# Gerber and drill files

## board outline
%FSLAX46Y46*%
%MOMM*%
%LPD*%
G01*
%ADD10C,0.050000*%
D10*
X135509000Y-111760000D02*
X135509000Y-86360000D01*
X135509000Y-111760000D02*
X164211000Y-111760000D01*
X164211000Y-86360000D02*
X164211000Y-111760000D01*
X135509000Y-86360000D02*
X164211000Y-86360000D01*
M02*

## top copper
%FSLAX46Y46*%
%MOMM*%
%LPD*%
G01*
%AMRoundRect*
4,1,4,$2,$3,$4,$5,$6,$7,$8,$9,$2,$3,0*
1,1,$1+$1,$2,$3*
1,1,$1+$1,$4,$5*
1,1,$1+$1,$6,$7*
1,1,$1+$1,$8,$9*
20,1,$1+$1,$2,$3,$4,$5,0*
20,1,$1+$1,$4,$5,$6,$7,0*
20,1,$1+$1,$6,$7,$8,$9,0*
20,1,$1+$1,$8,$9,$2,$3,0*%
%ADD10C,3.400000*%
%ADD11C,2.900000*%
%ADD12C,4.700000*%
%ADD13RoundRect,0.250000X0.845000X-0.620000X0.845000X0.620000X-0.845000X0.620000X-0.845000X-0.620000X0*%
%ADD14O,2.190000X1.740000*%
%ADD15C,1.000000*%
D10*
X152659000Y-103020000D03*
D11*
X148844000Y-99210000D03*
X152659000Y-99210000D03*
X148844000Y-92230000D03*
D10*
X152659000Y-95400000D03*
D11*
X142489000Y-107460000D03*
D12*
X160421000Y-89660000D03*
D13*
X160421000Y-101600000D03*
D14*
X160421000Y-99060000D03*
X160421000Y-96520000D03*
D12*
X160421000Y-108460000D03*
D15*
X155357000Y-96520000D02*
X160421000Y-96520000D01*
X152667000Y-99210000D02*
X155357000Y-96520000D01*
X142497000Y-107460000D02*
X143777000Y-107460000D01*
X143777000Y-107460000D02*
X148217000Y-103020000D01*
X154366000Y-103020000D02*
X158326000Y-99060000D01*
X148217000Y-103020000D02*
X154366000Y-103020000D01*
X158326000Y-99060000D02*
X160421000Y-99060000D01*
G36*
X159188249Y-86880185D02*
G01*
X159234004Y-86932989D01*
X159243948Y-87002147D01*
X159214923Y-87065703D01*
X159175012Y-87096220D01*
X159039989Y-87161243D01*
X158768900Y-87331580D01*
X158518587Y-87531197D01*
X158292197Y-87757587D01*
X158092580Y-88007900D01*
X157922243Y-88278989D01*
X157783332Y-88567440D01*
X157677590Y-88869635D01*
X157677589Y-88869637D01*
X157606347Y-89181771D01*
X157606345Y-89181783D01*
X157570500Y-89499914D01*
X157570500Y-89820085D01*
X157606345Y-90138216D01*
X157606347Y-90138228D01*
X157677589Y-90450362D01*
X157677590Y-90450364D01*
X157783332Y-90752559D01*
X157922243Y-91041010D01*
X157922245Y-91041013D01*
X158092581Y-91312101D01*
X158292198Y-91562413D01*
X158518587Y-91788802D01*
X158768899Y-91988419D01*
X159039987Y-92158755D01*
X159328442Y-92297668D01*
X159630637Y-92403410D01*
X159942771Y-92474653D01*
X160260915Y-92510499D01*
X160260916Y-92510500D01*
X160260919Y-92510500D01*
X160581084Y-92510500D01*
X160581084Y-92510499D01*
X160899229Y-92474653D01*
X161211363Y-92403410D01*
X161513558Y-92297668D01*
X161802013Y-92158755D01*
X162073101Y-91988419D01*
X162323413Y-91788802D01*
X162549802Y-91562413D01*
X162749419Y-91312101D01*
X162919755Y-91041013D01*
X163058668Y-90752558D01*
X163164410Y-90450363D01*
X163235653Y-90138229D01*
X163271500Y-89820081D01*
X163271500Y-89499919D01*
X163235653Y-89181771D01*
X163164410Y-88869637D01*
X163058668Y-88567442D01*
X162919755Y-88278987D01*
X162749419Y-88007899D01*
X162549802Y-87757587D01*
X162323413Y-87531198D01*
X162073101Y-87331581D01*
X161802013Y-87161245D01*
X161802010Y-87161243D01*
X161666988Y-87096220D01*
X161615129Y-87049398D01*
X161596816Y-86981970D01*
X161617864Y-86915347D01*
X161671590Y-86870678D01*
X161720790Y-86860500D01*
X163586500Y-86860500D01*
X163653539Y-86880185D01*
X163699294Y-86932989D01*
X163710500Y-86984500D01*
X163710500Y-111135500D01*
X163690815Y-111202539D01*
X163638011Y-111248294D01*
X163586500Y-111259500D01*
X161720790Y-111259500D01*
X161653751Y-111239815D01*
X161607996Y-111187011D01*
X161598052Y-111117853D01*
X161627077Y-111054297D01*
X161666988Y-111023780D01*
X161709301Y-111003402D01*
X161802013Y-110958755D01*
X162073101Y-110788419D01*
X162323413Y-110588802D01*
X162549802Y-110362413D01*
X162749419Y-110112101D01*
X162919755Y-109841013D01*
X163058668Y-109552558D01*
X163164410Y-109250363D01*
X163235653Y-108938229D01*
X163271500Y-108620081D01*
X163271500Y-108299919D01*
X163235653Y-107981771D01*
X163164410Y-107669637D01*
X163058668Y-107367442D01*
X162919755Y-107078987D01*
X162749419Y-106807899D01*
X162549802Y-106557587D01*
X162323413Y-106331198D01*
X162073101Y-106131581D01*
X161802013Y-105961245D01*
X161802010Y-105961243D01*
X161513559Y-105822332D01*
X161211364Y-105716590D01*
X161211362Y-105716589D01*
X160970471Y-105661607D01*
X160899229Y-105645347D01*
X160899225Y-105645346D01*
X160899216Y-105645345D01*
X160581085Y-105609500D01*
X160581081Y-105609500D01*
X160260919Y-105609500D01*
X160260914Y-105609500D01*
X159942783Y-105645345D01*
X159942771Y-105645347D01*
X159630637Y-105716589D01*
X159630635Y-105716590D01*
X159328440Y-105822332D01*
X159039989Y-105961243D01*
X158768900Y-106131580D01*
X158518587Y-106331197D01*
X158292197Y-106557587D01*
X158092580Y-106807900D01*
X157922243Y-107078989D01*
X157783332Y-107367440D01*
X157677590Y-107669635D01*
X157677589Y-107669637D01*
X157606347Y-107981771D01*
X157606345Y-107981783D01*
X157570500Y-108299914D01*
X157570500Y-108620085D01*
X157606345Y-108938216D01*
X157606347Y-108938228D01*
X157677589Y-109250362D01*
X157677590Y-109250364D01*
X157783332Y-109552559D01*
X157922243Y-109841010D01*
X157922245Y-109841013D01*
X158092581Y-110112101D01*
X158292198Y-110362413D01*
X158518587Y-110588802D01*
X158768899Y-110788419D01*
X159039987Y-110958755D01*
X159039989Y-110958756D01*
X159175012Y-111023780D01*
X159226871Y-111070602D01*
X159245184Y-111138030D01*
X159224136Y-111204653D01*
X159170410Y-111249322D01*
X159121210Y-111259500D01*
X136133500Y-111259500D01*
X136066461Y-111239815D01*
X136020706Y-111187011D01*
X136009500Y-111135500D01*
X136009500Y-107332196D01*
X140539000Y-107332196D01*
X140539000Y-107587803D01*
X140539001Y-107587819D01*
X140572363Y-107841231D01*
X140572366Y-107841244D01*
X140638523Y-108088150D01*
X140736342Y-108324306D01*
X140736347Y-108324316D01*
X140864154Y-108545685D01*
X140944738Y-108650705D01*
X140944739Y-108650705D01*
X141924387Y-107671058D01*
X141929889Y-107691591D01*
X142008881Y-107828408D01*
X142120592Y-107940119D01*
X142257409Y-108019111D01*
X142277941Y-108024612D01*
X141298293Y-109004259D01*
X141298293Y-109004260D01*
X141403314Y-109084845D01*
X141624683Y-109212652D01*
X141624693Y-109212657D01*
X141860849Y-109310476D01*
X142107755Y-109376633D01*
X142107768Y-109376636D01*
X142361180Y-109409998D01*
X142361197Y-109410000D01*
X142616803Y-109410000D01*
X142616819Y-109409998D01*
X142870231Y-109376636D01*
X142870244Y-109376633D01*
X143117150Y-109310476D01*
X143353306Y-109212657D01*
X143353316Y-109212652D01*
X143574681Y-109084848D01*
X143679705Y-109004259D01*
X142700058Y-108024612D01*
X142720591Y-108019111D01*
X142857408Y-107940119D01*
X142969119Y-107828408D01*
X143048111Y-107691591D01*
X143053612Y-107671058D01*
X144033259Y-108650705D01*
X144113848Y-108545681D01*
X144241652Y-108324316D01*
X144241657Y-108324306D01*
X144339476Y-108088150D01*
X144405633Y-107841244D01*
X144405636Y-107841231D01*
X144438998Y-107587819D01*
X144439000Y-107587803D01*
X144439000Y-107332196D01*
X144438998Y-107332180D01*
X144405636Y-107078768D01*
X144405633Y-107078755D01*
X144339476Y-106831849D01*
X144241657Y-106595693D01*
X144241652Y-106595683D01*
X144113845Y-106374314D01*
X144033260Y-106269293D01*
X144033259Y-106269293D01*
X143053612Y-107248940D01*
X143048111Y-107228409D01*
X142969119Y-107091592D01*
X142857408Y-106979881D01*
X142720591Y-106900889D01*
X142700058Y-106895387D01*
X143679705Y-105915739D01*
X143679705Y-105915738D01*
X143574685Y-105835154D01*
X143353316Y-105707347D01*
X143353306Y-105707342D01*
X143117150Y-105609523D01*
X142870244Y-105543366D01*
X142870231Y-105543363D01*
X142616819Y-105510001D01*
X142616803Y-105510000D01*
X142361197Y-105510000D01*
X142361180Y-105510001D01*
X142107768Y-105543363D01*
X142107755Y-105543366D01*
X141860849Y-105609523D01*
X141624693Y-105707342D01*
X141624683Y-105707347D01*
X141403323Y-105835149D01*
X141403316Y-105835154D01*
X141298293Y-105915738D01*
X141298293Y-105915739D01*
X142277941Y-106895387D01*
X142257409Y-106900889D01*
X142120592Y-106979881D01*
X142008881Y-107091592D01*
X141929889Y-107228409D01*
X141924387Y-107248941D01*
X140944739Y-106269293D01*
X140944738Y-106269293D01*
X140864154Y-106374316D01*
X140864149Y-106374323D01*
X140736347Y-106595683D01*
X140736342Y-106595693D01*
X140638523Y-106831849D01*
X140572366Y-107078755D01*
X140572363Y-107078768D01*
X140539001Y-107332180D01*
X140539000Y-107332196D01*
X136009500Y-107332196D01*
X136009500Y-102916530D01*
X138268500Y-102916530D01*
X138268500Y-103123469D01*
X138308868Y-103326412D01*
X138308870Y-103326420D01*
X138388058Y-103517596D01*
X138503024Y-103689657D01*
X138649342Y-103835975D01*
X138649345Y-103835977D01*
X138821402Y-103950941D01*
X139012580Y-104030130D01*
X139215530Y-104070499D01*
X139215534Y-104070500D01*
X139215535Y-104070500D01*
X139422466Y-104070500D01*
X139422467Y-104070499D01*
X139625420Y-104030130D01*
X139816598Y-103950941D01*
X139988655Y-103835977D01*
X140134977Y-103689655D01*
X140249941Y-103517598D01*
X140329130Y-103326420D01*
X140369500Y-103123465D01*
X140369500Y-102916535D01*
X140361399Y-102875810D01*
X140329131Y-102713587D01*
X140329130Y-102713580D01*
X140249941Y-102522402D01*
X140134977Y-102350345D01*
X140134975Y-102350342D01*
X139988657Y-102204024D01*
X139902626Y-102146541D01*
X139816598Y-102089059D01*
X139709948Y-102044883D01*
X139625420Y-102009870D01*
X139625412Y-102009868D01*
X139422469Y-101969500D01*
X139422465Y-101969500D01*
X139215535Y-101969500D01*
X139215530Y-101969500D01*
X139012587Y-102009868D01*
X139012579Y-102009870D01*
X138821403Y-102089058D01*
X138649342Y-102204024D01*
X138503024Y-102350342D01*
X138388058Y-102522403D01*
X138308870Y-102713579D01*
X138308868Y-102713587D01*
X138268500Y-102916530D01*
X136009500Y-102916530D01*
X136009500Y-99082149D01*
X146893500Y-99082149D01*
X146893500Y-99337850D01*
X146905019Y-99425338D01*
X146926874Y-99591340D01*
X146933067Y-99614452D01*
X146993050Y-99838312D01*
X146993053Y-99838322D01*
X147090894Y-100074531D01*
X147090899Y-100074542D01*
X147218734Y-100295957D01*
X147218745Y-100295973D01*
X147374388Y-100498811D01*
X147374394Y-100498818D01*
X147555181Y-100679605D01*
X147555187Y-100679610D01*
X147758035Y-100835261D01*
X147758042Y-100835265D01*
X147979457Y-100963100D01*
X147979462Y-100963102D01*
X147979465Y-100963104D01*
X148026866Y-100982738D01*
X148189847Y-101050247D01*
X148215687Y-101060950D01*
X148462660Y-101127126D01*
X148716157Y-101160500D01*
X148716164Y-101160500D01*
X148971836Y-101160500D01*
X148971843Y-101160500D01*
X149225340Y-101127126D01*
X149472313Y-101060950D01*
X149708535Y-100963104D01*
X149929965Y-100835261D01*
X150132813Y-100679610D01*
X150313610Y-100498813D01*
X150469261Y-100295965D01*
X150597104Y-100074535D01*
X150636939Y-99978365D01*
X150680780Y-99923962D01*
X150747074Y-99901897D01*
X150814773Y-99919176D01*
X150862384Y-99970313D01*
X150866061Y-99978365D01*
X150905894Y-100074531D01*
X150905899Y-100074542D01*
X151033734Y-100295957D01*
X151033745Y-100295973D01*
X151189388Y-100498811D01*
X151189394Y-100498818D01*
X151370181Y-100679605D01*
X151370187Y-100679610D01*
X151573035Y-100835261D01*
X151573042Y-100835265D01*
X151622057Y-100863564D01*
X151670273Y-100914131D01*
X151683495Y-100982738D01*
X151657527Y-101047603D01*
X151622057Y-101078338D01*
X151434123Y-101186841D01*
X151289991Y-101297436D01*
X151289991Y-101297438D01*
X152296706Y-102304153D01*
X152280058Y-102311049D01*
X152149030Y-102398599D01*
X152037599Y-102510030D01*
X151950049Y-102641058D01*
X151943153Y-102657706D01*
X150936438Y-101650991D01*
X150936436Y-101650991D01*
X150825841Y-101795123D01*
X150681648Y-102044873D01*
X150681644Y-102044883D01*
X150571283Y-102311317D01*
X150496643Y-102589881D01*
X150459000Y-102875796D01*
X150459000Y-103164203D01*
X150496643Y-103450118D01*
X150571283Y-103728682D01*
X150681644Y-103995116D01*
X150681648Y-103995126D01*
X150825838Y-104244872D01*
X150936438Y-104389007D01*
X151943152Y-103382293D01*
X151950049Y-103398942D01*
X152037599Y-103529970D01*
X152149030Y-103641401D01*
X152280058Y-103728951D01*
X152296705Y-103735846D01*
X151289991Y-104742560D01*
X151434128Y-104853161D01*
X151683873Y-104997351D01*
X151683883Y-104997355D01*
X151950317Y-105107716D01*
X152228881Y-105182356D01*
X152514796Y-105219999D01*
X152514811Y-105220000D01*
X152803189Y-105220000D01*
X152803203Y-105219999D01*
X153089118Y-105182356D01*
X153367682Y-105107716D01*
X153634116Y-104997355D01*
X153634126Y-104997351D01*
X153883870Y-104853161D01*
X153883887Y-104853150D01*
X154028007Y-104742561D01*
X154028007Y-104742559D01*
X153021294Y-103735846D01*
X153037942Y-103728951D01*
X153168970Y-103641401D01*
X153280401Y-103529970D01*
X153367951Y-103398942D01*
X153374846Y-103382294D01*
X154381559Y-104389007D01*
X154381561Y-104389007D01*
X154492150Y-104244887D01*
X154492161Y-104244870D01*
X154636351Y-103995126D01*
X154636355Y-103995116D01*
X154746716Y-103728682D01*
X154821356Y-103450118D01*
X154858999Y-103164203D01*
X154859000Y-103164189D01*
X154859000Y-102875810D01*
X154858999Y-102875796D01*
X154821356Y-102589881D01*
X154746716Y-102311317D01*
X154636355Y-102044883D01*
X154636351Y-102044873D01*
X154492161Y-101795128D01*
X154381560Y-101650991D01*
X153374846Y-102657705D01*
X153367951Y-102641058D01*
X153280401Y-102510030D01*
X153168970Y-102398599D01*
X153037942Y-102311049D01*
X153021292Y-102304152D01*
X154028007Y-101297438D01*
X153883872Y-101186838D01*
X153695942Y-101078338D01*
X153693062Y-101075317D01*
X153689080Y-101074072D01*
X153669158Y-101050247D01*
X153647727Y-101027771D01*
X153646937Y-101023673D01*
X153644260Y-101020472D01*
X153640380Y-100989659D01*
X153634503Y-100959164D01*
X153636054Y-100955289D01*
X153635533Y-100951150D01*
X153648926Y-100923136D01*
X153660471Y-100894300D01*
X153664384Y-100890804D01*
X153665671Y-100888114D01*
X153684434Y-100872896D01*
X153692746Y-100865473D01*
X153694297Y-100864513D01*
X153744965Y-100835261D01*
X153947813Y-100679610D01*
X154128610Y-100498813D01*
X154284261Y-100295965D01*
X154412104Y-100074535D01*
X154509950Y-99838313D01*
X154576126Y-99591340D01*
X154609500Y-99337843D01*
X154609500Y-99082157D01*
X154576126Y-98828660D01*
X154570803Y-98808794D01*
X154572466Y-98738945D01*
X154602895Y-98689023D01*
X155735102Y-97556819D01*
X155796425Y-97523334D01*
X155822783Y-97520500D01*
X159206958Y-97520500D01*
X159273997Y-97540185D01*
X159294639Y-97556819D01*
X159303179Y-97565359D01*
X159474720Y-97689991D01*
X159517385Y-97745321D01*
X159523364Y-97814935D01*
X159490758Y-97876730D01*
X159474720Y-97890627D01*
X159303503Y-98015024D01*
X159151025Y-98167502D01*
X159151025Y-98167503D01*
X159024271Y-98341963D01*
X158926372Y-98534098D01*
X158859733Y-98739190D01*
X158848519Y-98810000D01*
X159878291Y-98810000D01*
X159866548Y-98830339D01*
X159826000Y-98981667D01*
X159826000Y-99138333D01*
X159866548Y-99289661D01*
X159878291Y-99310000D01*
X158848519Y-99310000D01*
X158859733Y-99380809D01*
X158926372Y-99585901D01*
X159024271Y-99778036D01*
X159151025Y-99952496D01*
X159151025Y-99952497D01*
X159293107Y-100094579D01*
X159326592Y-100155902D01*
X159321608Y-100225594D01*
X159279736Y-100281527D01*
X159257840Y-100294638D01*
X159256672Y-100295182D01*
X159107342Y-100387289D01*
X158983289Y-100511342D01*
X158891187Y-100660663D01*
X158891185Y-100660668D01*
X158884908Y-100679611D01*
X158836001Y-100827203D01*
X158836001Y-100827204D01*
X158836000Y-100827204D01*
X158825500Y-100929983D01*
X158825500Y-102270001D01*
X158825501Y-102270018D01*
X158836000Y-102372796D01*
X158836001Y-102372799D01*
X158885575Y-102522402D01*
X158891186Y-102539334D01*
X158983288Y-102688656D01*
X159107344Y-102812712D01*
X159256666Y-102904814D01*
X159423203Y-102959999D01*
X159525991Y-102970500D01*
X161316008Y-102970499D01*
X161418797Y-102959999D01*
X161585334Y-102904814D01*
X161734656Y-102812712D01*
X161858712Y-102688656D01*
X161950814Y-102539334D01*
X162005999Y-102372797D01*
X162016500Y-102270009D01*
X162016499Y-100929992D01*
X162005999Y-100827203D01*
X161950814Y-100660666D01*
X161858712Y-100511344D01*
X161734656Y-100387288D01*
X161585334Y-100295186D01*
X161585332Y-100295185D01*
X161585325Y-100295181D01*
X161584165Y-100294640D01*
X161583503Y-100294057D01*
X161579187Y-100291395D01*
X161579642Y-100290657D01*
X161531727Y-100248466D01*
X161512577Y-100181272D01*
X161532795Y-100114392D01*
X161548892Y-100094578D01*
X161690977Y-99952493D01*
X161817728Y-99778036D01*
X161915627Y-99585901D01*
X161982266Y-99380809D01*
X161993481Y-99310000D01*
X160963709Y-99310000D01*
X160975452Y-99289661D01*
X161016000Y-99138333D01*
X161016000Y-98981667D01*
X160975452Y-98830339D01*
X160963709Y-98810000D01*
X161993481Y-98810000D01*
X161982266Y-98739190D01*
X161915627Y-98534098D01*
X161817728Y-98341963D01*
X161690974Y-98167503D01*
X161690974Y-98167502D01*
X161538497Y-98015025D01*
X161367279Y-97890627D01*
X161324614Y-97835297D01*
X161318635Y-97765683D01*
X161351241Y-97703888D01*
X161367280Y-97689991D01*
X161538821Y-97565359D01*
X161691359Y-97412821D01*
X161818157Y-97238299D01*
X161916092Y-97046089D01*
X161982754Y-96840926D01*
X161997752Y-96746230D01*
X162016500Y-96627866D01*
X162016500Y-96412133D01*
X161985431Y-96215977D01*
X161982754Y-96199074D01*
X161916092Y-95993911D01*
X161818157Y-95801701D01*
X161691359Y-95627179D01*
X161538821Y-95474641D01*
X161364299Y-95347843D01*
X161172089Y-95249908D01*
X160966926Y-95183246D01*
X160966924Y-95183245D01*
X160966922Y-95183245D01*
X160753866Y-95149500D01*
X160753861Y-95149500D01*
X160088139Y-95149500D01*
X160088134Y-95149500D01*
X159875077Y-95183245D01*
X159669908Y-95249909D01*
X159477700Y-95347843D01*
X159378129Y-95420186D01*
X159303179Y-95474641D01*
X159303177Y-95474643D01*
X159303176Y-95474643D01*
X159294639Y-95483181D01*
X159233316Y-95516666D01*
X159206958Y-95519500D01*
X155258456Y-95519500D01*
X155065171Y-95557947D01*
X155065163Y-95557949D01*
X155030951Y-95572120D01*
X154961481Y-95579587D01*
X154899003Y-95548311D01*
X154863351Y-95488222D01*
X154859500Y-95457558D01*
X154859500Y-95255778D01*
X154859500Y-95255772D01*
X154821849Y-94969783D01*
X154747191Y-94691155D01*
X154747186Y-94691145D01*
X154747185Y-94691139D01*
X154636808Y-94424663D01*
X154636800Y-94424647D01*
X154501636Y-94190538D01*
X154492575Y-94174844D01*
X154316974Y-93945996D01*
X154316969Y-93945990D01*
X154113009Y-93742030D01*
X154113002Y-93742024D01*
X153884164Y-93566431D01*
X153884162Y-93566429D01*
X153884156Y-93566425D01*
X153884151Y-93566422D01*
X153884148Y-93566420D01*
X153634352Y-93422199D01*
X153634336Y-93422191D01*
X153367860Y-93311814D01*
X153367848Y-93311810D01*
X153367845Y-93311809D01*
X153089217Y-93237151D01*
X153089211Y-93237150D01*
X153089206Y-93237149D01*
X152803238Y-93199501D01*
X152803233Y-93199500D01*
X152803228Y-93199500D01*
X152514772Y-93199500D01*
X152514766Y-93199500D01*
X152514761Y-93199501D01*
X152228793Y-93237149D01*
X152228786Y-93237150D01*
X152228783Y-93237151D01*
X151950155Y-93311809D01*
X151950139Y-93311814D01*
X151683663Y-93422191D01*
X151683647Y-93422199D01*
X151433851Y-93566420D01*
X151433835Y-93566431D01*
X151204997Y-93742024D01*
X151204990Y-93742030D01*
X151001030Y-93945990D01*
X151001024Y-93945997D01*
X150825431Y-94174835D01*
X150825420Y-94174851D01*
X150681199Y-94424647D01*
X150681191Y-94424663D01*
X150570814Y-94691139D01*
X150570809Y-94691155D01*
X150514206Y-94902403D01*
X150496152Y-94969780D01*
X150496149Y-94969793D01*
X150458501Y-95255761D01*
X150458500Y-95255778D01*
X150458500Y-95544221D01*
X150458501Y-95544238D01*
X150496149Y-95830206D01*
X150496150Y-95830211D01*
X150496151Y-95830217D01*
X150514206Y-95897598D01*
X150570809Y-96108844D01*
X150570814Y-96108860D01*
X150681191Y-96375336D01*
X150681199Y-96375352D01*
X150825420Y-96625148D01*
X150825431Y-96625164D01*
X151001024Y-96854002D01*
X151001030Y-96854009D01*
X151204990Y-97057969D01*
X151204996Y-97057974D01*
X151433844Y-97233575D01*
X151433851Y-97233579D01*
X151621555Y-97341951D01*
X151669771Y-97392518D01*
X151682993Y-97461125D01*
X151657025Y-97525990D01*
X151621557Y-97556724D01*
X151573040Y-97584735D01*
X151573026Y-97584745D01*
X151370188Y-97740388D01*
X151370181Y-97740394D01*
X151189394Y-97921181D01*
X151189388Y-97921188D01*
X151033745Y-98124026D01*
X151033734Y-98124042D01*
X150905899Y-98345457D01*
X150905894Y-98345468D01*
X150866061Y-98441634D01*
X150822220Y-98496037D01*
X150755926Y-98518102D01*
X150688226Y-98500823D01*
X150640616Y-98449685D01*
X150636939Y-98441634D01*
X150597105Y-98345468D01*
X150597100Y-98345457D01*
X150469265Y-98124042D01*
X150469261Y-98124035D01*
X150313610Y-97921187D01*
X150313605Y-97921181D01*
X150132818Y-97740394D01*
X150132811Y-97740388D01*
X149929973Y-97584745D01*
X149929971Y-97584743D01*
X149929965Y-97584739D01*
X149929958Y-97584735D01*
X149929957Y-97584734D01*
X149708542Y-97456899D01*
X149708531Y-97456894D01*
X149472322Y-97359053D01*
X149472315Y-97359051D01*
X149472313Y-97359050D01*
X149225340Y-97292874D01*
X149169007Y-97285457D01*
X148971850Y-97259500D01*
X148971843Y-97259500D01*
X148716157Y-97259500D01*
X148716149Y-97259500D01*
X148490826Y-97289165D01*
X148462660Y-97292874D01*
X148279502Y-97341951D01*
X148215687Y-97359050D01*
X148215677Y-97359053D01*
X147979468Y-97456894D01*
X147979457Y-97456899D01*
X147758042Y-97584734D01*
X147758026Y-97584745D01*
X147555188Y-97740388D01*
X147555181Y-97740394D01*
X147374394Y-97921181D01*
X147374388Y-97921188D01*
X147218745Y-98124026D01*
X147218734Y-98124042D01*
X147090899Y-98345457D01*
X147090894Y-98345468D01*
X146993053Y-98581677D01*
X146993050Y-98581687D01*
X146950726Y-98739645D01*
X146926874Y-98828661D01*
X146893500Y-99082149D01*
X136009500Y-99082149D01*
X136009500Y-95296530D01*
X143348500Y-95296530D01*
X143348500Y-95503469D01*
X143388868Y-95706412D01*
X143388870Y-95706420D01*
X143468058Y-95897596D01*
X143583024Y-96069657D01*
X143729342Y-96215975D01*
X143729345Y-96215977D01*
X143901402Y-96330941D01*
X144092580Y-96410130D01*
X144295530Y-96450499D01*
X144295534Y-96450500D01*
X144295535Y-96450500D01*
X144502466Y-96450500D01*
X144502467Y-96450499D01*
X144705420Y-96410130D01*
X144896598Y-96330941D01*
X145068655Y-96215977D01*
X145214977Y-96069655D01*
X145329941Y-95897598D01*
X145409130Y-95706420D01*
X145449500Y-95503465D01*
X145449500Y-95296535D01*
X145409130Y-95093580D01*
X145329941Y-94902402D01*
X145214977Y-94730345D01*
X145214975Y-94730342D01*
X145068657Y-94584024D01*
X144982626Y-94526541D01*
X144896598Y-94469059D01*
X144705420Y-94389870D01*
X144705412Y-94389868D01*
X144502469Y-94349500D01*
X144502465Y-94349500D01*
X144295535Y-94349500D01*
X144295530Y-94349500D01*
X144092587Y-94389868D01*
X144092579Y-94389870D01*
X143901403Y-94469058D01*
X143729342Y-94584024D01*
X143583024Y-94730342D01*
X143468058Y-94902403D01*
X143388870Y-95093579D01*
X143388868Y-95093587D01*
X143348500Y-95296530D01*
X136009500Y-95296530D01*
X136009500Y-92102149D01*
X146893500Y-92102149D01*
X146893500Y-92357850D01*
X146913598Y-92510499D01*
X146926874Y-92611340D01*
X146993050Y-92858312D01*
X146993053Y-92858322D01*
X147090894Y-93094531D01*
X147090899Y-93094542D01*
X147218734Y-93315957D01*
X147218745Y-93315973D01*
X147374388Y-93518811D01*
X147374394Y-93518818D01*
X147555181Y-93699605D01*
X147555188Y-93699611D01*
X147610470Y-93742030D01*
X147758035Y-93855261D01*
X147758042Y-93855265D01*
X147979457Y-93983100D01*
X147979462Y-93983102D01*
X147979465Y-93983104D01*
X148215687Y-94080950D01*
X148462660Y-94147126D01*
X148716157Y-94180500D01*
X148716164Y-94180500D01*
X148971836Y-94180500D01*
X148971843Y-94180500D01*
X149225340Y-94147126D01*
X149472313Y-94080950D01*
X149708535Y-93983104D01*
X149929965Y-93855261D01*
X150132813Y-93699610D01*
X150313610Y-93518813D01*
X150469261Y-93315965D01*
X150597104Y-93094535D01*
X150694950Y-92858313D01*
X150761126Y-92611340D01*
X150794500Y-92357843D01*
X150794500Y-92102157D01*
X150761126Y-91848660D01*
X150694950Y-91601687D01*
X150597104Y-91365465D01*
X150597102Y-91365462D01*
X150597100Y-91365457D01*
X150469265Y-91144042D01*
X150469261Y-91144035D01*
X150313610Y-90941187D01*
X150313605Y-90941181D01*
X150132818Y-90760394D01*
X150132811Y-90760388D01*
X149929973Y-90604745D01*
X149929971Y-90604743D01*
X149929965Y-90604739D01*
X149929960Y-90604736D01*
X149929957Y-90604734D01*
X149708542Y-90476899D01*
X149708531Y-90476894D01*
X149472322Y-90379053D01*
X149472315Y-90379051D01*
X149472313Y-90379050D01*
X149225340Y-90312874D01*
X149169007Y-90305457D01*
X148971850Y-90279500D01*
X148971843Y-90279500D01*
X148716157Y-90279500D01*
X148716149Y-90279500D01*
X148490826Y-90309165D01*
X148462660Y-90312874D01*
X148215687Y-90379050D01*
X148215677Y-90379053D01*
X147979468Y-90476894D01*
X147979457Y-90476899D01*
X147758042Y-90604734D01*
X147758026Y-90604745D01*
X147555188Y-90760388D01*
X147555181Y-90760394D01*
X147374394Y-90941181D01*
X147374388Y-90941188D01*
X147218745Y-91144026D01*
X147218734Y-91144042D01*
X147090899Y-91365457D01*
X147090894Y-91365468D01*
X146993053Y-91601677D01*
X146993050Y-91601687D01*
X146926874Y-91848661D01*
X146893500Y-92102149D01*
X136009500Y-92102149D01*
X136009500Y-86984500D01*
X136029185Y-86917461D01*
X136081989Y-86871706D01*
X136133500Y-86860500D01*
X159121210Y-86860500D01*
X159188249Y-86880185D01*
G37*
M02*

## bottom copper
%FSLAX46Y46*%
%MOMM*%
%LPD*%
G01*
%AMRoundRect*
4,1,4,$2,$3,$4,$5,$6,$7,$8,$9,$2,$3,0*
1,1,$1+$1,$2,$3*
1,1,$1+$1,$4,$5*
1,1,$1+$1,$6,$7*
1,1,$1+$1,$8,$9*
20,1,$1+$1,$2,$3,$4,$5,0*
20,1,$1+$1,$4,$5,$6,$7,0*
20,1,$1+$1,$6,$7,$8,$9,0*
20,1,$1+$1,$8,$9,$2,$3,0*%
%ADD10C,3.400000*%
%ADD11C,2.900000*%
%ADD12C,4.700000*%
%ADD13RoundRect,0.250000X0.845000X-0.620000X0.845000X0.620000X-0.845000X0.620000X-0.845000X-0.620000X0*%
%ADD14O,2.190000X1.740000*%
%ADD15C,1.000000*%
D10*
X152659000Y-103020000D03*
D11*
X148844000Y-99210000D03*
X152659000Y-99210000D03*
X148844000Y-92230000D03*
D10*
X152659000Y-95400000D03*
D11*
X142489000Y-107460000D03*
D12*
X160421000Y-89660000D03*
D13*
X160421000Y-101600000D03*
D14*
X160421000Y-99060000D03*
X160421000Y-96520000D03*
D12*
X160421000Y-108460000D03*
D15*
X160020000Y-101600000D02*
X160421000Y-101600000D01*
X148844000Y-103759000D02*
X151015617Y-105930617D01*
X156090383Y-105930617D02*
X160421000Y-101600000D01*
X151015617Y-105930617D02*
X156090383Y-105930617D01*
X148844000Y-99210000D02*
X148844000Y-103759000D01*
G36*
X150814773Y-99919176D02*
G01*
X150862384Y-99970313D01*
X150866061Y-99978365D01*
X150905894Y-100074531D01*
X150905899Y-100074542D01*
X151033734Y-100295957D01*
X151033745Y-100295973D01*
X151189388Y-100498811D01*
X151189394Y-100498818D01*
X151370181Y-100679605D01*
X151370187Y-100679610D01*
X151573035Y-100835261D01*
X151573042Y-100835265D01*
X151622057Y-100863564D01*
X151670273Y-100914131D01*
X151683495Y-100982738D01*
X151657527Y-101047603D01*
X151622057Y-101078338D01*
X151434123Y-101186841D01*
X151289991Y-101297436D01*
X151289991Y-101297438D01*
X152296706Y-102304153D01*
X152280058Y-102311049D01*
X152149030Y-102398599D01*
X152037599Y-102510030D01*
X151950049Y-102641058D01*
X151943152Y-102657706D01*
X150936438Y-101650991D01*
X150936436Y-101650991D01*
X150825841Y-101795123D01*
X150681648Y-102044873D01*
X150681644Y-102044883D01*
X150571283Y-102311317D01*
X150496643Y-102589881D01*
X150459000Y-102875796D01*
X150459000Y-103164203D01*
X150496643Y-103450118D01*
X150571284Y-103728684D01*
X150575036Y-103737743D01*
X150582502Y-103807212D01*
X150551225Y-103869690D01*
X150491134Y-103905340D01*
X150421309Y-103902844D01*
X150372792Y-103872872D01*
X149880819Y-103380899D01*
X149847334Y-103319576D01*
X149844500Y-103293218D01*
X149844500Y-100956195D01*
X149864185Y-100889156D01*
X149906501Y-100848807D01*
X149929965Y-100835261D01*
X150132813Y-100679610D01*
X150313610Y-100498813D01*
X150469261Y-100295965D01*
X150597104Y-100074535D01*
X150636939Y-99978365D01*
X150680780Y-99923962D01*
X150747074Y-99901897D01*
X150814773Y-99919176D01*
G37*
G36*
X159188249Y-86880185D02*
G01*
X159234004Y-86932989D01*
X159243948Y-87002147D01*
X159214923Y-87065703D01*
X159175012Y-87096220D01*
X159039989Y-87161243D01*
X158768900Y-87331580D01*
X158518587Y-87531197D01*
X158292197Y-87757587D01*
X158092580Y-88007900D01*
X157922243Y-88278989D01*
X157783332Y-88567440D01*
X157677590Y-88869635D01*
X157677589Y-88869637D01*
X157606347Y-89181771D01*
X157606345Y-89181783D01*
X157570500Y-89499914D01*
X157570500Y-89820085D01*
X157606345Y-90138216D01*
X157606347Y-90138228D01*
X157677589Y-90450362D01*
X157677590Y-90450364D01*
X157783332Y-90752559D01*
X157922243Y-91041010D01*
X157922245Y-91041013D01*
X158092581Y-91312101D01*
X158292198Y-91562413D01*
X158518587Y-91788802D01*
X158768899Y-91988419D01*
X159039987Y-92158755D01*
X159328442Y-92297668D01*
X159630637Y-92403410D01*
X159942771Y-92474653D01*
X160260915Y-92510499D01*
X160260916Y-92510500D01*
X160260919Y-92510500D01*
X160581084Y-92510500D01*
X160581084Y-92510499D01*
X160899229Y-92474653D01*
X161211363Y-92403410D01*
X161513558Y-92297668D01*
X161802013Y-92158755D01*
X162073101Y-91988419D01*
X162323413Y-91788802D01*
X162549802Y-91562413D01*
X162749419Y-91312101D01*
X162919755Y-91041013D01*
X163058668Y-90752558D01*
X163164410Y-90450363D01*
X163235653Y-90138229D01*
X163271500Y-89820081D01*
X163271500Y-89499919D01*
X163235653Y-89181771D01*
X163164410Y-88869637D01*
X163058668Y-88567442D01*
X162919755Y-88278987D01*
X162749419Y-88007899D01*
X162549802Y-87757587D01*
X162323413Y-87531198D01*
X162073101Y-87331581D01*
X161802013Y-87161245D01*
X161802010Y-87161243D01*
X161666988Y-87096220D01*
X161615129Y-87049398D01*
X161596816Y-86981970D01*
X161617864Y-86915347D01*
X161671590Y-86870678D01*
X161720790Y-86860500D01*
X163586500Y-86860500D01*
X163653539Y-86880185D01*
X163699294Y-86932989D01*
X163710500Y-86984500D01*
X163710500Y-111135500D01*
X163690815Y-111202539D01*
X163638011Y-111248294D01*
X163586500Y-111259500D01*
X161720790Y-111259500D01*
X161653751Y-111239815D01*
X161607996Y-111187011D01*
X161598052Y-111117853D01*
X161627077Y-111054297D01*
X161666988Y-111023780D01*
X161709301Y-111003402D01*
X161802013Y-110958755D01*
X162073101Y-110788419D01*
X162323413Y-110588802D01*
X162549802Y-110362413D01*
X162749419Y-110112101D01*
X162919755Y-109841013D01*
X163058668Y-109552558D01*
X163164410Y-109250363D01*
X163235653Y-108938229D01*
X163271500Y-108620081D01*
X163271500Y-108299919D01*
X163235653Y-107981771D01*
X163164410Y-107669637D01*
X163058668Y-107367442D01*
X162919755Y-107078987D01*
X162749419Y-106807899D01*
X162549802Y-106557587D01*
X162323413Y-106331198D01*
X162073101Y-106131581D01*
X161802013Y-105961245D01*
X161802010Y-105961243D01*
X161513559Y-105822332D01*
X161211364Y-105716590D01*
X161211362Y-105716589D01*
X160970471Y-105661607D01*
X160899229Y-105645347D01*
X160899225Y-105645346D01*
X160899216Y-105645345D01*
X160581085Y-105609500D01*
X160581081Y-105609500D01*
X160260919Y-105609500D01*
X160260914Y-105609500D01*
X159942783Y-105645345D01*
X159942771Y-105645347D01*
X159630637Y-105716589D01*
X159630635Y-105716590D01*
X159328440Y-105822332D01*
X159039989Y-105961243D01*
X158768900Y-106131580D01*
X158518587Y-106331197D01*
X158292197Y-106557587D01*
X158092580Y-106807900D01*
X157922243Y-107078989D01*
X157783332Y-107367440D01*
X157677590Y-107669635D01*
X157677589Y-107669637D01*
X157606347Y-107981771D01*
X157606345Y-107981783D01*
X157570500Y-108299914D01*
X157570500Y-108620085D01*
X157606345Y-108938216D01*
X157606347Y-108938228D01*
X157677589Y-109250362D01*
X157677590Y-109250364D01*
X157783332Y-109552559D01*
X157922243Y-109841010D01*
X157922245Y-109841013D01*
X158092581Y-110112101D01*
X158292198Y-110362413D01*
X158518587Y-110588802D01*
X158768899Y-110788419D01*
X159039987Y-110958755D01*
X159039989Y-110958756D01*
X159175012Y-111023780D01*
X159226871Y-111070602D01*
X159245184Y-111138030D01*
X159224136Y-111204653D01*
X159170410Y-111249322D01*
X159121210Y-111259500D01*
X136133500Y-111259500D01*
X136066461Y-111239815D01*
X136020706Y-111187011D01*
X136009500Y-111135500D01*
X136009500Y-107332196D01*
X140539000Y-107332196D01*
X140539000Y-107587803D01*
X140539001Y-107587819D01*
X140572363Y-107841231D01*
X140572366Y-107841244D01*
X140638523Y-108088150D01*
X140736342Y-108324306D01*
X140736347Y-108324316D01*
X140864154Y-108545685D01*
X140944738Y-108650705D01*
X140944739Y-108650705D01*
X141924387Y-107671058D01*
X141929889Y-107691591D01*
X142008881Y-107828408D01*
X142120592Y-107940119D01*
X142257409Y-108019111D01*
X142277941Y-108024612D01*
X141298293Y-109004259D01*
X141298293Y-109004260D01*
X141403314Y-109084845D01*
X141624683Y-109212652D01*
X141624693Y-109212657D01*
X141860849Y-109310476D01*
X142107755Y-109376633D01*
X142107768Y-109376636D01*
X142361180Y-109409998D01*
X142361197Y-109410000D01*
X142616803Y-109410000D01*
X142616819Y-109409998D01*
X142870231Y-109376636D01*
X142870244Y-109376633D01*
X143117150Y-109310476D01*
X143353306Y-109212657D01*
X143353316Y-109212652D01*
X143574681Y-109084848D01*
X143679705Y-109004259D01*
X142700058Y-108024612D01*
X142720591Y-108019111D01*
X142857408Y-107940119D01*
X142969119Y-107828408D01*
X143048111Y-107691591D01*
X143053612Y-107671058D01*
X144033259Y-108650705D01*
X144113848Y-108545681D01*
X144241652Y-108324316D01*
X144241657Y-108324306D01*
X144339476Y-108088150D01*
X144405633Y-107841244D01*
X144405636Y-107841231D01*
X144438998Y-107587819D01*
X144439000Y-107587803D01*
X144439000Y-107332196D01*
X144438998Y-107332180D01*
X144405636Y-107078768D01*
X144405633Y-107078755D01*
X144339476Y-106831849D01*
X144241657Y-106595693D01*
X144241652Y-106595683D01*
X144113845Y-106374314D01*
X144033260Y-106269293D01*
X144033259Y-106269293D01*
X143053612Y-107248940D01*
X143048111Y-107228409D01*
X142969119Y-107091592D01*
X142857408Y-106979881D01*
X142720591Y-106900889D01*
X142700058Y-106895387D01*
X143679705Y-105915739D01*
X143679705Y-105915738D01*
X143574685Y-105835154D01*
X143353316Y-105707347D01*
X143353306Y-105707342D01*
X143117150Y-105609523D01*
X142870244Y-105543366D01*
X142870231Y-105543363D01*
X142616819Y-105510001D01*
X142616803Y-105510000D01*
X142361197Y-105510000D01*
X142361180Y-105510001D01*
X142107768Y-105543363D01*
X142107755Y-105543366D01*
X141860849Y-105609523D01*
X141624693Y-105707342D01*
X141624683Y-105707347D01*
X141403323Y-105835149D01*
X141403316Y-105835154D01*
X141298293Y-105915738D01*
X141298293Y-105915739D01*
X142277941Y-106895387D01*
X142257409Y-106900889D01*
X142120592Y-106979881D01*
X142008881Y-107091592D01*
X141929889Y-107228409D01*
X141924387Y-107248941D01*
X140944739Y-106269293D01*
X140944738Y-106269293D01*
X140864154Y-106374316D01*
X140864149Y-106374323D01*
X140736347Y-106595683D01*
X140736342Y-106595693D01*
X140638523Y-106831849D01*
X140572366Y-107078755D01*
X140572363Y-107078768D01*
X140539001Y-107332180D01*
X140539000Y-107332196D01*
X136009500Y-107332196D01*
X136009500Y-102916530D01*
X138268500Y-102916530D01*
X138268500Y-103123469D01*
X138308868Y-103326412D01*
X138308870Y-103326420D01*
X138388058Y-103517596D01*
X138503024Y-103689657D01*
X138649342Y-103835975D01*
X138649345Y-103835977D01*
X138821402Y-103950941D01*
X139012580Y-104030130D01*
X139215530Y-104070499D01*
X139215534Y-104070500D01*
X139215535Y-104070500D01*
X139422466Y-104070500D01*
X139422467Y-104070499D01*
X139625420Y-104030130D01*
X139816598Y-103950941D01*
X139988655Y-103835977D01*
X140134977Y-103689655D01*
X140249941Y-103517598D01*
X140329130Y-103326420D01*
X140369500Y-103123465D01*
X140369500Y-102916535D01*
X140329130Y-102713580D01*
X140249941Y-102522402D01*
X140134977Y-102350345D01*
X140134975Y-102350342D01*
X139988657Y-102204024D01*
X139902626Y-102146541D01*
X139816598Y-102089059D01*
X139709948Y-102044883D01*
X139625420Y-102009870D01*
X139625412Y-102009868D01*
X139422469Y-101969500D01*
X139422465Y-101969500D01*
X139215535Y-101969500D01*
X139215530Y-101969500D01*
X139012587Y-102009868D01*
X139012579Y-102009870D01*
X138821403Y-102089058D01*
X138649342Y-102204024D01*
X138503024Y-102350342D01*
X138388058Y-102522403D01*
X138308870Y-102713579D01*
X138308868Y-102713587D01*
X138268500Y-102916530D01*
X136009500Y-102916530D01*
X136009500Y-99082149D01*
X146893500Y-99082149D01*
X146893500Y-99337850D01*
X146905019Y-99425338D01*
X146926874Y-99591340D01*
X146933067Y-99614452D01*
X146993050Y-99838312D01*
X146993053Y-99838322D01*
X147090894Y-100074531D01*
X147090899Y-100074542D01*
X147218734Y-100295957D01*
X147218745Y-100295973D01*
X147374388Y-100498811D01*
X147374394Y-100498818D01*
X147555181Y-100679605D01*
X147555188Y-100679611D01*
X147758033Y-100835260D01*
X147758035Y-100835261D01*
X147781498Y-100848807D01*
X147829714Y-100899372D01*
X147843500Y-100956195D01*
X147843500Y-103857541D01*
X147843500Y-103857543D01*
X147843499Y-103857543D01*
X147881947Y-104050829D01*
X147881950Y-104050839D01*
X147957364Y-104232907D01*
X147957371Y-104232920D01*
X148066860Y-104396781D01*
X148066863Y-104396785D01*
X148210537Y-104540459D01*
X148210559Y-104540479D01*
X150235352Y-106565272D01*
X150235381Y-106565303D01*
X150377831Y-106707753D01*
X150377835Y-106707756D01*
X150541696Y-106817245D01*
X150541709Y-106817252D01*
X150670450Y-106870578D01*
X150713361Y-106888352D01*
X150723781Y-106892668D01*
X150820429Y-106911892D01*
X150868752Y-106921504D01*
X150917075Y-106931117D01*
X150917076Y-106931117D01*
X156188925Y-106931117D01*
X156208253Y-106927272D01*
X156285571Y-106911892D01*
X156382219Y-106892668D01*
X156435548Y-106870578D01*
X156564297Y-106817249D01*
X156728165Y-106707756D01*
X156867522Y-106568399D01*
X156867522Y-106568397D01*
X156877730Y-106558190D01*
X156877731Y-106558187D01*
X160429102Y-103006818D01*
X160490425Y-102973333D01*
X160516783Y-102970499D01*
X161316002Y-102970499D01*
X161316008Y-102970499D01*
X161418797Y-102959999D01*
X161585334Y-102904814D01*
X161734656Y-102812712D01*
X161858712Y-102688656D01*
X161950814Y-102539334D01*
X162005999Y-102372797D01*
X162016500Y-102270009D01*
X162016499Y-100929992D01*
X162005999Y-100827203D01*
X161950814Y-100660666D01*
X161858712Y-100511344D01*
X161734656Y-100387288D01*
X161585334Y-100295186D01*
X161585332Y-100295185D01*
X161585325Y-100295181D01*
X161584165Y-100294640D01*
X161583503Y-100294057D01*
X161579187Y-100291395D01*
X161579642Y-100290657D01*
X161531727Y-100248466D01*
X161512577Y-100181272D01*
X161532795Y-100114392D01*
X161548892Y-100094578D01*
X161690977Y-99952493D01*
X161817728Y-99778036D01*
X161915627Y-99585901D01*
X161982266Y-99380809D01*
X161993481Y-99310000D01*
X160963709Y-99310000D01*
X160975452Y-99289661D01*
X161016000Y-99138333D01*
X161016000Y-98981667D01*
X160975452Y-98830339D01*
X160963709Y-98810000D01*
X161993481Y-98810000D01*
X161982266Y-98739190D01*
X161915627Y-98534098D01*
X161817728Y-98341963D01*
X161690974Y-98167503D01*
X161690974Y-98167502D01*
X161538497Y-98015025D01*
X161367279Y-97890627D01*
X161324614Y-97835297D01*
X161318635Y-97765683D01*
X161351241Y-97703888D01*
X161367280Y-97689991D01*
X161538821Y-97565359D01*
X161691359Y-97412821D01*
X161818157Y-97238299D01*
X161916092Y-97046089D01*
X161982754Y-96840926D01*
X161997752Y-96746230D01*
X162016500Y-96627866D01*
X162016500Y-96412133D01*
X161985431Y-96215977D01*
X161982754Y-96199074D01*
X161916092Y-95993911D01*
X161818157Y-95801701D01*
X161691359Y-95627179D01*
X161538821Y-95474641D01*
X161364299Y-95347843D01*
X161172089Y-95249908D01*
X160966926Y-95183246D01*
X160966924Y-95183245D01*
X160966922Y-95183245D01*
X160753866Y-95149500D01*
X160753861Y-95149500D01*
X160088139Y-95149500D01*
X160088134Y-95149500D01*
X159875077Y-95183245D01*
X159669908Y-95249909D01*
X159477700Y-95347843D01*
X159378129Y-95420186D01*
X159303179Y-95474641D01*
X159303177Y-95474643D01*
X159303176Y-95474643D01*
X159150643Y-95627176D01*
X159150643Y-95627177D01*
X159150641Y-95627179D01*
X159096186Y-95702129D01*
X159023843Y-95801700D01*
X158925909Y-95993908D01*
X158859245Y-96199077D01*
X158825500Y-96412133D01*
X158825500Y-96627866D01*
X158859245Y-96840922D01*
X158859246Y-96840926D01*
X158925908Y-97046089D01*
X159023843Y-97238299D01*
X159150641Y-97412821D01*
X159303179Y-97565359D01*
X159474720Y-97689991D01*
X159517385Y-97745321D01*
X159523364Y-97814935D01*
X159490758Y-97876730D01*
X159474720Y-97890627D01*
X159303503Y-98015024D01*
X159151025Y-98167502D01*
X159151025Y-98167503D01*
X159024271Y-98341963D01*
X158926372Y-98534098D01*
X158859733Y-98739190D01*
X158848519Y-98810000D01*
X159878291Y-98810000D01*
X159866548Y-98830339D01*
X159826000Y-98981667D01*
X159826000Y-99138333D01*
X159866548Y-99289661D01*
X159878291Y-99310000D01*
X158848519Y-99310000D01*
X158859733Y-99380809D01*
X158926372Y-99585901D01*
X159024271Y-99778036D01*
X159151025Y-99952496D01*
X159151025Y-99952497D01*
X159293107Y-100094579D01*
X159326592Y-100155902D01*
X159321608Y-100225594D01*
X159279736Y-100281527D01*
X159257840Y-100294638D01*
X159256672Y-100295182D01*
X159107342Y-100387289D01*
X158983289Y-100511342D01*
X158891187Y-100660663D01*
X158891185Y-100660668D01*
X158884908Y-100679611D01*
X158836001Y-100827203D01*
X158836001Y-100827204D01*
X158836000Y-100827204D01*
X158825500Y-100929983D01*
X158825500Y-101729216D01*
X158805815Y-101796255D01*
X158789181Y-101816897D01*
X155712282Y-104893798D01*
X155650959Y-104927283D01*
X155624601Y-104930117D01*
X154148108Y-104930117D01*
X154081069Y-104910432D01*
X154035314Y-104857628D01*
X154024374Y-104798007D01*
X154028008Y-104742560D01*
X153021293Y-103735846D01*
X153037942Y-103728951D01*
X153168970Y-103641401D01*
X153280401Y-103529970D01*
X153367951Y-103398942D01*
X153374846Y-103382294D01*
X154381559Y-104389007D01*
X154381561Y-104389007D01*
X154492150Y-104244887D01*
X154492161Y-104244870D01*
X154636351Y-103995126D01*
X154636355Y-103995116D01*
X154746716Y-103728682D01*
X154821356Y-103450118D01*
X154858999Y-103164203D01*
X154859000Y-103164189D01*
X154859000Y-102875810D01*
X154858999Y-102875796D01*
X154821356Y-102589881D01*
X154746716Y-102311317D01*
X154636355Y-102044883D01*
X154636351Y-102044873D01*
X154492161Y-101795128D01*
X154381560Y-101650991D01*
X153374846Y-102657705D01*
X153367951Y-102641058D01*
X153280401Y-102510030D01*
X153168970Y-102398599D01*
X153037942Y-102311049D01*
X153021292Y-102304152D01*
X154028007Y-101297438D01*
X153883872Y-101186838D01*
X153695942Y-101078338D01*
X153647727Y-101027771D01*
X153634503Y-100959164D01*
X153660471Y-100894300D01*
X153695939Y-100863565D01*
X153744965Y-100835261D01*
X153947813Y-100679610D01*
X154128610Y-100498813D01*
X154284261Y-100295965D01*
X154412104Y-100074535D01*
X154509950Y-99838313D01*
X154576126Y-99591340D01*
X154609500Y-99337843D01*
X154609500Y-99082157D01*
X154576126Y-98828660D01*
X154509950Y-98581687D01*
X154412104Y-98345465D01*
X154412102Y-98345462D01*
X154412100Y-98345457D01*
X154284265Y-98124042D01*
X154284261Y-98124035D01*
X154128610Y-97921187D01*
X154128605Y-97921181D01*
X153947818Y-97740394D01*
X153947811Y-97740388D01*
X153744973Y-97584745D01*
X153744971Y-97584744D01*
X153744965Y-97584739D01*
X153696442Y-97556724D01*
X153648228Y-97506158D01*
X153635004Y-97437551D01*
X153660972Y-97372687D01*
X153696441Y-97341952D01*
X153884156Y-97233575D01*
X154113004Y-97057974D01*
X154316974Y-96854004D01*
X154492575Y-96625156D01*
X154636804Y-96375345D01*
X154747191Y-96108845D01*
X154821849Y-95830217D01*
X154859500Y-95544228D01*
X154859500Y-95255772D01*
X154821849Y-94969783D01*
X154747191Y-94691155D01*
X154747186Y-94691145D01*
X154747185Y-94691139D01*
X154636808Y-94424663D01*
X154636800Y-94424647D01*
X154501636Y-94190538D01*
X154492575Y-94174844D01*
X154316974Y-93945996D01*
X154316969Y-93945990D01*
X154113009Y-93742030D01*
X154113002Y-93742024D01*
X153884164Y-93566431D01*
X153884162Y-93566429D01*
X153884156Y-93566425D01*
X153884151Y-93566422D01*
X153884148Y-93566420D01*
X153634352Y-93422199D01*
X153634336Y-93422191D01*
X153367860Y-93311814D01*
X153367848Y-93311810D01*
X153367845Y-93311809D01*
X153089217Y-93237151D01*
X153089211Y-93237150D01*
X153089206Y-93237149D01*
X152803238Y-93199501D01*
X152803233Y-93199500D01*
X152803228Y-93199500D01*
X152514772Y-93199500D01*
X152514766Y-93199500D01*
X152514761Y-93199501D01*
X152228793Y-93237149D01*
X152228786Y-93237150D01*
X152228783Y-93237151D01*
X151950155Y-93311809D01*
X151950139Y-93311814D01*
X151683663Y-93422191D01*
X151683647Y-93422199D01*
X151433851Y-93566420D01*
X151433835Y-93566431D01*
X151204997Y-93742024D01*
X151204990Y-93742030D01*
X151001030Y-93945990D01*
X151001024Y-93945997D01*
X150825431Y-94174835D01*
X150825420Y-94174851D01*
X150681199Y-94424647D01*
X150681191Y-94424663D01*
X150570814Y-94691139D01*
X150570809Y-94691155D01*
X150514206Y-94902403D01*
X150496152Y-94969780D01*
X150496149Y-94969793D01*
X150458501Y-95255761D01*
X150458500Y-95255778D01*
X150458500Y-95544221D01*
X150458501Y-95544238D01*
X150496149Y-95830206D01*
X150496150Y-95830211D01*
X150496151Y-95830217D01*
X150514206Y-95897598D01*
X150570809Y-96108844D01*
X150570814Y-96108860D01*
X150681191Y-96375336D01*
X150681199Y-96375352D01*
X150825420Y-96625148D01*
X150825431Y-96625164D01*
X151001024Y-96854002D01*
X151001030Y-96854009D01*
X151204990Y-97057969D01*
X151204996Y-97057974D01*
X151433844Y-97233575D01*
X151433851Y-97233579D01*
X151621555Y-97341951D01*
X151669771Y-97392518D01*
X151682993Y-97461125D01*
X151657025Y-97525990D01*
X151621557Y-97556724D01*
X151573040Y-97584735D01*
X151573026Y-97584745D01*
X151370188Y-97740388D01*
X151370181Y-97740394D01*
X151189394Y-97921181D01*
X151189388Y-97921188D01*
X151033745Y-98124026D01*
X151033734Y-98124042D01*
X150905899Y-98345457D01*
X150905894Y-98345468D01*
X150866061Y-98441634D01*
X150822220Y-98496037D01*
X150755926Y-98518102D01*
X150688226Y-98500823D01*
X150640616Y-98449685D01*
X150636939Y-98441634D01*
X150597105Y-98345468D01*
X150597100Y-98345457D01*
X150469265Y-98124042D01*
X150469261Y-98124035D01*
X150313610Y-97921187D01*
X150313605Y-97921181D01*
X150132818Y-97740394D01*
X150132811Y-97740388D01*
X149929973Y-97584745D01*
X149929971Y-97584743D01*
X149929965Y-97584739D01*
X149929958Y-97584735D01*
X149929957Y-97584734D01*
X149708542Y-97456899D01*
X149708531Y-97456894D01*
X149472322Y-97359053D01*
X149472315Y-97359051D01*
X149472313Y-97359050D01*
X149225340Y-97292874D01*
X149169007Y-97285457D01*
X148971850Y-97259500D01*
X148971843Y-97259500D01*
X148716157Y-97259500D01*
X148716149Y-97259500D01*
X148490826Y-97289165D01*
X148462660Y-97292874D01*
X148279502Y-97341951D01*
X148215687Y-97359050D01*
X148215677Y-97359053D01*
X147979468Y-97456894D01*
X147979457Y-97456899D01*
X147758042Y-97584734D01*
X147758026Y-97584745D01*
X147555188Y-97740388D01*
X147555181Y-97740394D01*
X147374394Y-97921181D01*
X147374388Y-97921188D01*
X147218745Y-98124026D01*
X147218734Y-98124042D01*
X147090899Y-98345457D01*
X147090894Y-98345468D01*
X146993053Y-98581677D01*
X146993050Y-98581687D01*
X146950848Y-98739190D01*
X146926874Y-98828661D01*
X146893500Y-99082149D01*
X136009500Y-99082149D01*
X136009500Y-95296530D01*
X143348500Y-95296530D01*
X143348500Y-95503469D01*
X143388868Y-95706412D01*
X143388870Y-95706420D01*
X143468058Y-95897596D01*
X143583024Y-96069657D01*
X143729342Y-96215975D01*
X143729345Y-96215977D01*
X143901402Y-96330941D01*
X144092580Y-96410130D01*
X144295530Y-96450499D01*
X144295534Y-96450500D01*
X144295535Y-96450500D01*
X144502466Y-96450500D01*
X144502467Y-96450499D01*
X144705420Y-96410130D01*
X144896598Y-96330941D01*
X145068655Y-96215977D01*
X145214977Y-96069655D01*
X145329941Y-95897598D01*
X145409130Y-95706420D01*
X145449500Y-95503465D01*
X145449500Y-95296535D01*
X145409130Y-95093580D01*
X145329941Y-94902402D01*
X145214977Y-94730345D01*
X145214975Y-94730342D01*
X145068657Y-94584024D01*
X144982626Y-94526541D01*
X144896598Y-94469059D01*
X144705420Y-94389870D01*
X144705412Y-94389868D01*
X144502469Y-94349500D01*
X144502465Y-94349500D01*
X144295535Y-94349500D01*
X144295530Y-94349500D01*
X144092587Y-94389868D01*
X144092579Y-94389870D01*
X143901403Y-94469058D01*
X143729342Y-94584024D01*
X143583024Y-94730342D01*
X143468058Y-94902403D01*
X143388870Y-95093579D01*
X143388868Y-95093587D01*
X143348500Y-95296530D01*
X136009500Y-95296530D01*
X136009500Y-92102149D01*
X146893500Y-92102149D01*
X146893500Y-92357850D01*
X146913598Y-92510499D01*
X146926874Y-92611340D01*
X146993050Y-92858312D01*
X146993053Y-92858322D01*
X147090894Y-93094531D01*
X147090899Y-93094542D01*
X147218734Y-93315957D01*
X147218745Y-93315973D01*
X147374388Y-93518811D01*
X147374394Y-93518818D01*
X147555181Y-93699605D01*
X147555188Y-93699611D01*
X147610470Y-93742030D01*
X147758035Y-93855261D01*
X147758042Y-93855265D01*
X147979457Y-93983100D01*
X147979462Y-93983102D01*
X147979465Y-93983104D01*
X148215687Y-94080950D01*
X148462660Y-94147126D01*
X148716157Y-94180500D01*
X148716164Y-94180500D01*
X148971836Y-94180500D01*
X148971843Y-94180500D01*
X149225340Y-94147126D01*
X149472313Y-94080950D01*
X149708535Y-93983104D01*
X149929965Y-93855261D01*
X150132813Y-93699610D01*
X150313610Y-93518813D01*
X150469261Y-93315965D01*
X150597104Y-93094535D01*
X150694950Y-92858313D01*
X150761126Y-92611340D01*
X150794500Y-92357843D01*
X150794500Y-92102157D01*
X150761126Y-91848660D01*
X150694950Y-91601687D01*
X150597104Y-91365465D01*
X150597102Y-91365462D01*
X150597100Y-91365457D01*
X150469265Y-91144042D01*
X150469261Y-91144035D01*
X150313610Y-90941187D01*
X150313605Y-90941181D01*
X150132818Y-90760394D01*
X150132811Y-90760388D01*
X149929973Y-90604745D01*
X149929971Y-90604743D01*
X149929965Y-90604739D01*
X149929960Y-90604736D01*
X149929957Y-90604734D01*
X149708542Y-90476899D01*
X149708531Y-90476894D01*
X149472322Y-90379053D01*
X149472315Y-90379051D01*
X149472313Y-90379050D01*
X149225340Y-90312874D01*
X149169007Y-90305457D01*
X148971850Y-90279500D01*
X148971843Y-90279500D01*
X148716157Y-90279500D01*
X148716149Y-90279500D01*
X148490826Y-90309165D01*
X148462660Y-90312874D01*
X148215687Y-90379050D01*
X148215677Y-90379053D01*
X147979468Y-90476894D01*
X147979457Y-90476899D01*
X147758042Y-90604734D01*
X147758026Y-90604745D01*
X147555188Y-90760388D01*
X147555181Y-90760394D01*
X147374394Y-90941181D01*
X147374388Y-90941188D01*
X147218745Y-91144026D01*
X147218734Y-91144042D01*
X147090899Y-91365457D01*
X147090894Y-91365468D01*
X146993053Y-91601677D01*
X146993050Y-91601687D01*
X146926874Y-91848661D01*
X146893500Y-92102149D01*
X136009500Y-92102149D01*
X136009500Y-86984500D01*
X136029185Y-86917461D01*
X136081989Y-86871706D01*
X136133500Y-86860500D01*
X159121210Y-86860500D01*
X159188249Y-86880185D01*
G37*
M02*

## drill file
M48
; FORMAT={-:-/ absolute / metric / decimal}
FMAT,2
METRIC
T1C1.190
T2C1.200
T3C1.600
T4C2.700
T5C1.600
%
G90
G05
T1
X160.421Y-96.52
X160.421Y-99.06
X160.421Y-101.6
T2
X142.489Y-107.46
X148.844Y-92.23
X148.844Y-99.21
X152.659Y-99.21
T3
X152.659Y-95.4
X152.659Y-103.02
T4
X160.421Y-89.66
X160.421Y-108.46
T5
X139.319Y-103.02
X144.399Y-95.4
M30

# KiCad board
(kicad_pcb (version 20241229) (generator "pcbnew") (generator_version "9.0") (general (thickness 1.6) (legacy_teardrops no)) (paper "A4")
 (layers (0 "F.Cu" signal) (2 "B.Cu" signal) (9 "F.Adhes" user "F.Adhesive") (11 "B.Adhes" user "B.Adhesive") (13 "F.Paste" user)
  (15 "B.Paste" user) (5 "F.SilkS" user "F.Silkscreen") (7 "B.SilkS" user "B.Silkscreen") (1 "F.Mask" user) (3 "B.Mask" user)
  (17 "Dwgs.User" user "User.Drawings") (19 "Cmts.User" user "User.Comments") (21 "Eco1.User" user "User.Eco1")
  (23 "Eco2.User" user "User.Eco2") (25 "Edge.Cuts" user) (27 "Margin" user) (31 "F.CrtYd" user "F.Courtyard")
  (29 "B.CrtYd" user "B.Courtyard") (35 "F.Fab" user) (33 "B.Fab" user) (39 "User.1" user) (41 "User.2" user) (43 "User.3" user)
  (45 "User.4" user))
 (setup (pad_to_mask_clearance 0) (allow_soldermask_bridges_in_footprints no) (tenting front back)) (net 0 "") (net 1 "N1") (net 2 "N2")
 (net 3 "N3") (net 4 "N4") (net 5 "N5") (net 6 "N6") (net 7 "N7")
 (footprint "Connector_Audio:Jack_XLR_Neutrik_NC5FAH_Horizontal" (layer "F.Cu") (at 152.659 103.02 180)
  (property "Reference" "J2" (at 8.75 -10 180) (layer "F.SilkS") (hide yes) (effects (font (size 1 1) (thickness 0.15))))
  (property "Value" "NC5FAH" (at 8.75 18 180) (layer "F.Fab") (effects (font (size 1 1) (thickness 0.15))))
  (pad "" np_thru_hole circle (at 8.26 7.62 180) (size 1.6 1.6) (drill 1.6) (layers "*.Cu" "*.Mask"))
  (pad "" np_thru_hole circle (at 13.34 0 180) (size 1.6 1.6) (drill 1.6) (layers "*.Cu" "*.Mask"))
  (pad "1" thru_hole circle (at 0 0 180) (size 3.4 3.4) (drill 1.6) (layers "*.Cu" "*.Mask") (remove_unused_layers no) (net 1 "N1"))
  (pad "2" thru_hole circle (at 3.815 3.81 180) (size 2.9 2.9) (drill 1.2) (layers "*.Cu" "*.Mask") (remove_unused_layers no) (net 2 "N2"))
  (pad "3" thru_hole circle (at 0 3.81 180) (size 2.9 2.9) (drill 1.2) (layers "*.Cu" "*.Mask") (remove_unused_layers no) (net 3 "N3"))
  (pad "4" thru_hole circle (at 3.815 10.79 180) (size 2.9 2.9) (drill 1.2) (layers "*.Cu" "*.Mask") (remove_unused_layers no) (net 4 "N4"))
  (pad "5" thru_hole circle (at 0 7.62 180) (size 3.4 3.4) (drill 1.6) (layers "*.Cu" "*.Mask") (remove_unused_layers no) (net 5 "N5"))
  (pad "G" thru_hole circle (at 10.17 -4.44 180) (size 2.9 2.9) (drill 1.2) (layers "*.Cu" "*.Mask") (remove_unused_layers no) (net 1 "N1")))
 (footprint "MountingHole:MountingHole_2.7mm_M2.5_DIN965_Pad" (layer "F.Cu") (at 160.421 89.66)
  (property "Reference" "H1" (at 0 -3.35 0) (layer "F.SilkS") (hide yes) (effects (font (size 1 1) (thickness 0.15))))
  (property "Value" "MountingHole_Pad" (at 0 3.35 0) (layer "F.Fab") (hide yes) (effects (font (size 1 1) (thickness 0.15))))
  (pad "1" thru_hole circle (at 0 0) (size 4.7 4.7) (drill 2.7) (layers "*.Cu" "*.Mask") (remove_unused_layers no) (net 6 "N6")))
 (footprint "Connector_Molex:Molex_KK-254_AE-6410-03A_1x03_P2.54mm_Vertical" (layer "F.Cu") (at 160.421 101.6 90)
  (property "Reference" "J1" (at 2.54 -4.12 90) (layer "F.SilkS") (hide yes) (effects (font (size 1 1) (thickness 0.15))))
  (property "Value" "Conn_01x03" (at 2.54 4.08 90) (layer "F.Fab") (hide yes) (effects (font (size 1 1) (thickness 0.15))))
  (pad "1" thru_hole roundrect (at 0 0 90) (size 1.74 2.19) (drill 1.19) (layers "*.Cu" "*.Mask") (remove_unused_layers no)
   (roundrect_rratio 0.143678) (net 2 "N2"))
  (pad "2" thru_hole oval (at 2.54 0 90) (size 1.74 2.19) (drill 1.19) (layers "*.Cu" "*.Mask") (remove_unused_layers no) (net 1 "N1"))
  (pad "3" thru_hole oval (at 5.08 0 90) (size 1.74 2.19) (drill 1.19) (layers "*.Cu" "*.Mask") (remove_unused_layers no) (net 3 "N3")))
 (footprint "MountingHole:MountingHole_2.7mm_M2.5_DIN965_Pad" (layer "F.Cu") (at 160.401 108.46)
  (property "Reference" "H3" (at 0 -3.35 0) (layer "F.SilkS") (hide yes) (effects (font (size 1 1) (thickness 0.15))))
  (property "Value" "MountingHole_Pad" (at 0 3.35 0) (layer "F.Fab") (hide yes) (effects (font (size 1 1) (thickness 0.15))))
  (pad "1" thru_hole circle (at 0.02 0) (size 4.7 4.7) (drill 2.7) (layers "*.Cu" "*.Mask") (remove_unused_layers no) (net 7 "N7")))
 (gr_line (start 135.509 111.76) (end 135.509 86.36) (stroke (width 0.05) (type default)) (layer "Edge.Cuts"))
 (gr_line (start 135.509 111.76) (end 164.211 111.76) (stroke (width 0.05) (type default)) (layer "Edge.Cuts"))
 (gr_line (start 164.211 86.36) (end 164.211 111.76) (stroke (width 0.05) (type default)) (layer "Edge.Cuts"))
 (gr_line (start 135.509 86.36) (end 164.211 86.36) (stroke (width 0.05) (type default)) (layer "Edge.Cuts"))
 (segment (start 155.357 96.52) (end 160.421 96.52) (width 1) (layer "F.Cu") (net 3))
 (segment (start 152.667 99.21) (end 155.357 96.52) (width 1) (layer "F.Cu") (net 3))
 (segment (start 160.02 101.6) (end 160.421 101.6) (width 1) (layer "B.Cu") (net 2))
 (segment (start 148.844 103.759) (end 151.015617 105.930617) (width 1) (layer "B.Cu") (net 2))
 (segment (start 156.090383 105.930617) (end 160.421 101.6) (width 1) (layer "B.Cu") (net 2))
 (segment (start 151.015617 105.930617) (end 156.090383 105.930617) (width 1) (layer "B.Cu") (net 2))
 (segment (start 148.844 99.21) (end 148.844 103.759) (width 1) (layer "B.Cu") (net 2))
 (segment (start 142.497 107.46) (end 143.777 107.46) (width 1) (layer "F.Cu") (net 1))
 (segment (start 143.777 107.46) (end 148.217 103.02) (width 1) (layer "F.Cu") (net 1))
 (segment (start 154.366 103.02) (end 158.326 99.06) (width 1) (layer "F.Cu") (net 1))
 (segment (start 148.217 103.02) (end 154.366 103.02) (width 1) (layer "F.Cu") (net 1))
 (segment (start 158.326 99.06) (end 160.421 99.06) (width 1) (layer "F.Cu") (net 1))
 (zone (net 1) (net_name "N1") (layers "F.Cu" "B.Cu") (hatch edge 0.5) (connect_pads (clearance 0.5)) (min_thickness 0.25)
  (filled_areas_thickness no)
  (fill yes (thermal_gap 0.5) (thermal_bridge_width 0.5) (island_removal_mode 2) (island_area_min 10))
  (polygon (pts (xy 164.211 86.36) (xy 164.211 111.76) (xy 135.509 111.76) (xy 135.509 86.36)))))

